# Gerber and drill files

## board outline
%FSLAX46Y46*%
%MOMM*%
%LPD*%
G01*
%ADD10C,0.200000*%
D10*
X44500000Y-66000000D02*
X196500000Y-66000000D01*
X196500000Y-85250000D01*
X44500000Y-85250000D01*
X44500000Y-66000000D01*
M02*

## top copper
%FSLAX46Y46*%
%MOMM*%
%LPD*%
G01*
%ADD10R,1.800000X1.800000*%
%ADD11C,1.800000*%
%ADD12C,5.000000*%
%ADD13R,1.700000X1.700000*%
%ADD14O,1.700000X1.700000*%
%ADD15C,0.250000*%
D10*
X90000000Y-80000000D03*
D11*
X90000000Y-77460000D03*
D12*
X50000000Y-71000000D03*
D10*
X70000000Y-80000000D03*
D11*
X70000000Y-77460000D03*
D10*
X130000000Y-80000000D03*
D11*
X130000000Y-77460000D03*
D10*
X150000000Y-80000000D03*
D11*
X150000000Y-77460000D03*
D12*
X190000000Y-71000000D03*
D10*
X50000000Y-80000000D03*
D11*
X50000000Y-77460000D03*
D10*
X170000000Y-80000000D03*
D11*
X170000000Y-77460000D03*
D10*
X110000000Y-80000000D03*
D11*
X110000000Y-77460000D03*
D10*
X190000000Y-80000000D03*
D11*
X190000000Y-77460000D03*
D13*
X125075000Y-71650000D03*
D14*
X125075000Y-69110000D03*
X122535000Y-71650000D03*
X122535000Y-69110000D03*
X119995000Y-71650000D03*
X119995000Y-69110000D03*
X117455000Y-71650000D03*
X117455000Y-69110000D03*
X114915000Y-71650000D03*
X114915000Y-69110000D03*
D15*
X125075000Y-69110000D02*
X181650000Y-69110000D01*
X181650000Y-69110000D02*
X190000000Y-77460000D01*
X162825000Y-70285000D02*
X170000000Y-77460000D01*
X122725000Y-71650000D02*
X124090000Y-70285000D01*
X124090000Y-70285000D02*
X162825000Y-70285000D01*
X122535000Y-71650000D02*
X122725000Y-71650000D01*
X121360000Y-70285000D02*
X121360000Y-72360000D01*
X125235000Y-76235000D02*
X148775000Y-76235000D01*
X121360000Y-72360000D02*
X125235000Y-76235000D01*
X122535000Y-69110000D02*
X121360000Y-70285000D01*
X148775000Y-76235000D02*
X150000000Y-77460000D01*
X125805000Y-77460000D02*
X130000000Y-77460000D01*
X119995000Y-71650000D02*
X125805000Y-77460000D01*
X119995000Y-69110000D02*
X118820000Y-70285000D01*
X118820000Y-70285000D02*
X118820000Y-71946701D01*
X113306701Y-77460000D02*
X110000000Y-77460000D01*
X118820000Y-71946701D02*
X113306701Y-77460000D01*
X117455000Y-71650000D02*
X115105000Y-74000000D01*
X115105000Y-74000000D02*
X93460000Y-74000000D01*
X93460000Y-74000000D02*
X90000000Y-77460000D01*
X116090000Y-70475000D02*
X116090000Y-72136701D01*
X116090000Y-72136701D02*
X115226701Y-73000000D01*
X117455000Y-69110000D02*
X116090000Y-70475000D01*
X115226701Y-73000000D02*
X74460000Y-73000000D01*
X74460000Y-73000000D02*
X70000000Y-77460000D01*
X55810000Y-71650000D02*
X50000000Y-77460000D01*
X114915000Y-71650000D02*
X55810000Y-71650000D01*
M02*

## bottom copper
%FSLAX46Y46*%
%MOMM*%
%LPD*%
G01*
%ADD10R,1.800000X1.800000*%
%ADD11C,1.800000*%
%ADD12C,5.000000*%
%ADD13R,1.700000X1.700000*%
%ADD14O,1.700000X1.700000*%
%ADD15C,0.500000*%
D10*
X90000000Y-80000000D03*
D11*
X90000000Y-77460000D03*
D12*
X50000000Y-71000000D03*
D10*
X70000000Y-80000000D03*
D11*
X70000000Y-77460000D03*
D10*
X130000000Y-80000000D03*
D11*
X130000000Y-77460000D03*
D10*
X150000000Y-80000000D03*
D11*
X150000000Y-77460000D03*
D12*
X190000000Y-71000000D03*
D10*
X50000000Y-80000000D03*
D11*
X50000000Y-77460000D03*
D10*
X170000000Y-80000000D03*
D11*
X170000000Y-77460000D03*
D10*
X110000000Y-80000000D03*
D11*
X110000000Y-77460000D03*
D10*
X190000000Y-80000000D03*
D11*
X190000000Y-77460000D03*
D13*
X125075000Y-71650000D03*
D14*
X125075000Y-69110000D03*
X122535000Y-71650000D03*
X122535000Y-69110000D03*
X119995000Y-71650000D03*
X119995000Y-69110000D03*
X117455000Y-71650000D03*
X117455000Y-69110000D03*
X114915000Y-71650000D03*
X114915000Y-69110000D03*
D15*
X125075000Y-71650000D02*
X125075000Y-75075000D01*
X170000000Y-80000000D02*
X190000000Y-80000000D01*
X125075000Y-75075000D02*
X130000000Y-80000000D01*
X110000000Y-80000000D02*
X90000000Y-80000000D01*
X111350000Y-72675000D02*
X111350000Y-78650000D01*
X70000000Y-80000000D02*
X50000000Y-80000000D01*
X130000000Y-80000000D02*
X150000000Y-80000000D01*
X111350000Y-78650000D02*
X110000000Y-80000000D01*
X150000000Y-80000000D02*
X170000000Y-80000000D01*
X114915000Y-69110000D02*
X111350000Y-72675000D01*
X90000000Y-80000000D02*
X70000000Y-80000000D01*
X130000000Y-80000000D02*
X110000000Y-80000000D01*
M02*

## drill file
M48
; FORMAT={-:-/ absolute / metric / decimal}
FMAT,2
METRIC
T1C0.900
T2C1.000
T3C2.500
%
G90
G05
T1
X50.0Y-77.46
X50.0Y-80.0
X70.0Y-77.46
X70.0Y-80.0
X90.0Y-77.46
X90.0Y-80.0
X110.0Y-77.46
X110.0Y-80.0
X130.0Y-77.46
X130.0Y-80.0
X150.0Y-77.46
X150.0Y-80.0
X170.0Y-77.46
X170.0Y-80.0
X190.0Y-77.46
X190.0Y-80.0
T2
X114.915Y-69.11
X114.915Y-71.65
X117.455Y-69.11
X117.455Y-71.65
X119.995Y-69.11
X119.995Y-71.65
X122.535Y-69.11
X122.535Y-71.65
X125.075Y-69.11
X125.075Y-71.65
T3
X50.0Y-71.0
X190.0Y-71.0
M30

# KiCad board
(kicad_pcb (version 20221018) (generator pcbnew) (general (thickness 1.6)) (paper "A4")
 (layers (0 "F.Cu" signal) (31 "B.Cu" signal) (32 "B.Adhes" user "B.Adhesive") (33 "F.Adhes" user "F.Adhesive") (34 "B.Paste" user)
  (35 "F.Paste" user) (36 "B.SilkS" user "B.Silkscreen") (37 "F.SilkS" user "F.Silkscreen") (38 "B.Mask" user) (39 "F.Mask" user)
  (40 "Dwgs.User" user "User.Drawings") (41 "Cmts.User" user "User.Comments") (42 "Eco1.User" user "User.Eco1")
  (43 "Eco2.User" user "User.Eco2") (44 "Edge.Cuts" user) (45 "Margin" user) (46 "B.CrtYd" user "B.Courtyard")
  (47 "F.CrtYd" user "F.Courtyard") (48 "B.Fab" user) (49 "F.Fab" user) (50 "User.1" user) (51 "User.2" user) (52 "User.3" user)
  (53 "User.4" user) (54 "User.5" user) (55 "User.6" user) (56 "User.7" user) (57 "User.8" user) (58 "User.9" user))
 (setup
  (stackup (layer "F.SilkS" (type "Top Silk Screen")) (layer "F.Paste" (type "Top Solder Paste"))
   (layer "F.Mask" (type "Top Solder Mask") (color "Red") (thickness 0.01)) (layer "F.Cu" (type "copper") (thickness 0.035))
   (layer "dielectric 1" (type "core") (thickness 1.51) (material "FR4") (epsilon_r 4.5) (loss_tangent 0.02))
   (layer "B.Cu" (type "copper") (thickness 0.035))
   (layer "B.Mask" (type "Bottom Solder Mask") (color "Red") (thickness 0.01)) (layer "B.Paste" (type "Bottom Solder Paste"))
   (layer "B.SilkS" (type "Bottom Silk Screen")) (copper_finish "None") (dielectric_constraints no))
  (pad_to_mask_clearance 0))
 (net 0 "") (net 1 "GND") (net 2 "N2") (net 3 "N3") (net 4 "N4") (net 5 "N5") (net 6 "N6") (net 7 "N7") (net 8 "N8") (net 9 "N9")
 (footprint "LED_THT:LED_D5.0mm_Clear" (layer "F.Cu") (at 90 80 90)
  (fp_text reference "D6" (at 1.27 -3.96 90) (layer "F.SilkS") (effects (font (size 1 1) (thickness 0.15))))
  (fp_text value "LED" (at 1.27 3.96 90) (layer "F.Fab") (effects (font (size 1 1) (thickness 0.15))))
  (pad "1" thru_hole rect (at 0 0 90) (size 1.8 1.8) (drill 0.9) (layers "*.Cu" "*.Mask") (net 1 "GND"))
  (pad "2" thru_hole circle (at 2.54 0 90) (size 1.8 1.8) (drill 0.9) (layers "*.Cu" "*.Mask") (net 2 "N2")))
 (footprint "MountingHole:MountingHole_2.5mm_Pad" (layer "F.Cu") (at 50 71)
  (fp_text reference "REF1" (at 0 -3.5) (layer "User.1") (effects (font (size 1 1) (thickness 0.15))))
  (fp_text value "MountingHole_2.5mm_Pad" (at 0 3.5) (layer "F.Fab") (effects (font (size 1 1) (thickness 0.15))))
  (pad "1" thru_hole circle (at 0 0) (size 5 5) (drill 2.5) (layers "*.Cu" "*.Mask")))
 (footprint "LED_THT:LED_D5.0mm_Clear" (layer "F.Cu") (at 70 80 90)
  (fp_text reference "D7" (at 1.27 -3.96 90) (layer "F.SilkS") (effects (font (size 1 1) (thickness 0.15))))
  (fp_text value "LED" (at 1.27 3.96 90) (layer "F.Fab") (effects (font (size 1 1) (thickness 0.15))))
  (pad "1" thru_hole rect (at 0 0 90) (size 1.8 1.8) (drill 0.9) (layers "*.Cu" "*.Mask") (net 1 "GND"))
  (pad "2" thru_hole circle (at 2.54 0 90) (size 1.8 1.8) (drill 0.9) (layers "*.Cu" "*.Mask") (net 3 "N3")))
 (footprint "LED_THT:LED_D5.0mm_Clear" (layer "F.Cu") (at 130 80 90)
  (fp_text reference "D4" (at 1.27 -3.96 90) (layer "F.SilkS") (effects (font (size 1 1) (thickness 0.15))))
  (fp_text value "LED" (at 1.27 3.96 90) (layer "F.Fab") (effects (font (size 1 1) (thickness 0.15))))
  (pad "1" thru_hole rect (at 0 0 90) (size 1.8 1.8) (drill 0.9) (layers "*.Cu" "*.Mask") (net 1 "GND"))
  (pad "2" thru_hole circle (at 2.54 0 90) (size 1.8 1.8) (drill 0.9) (layers "*.Cu" "*.Mask") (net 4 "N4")))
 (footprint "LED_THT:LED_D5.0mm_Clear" (layer "F.Cu") (at 150 80 90)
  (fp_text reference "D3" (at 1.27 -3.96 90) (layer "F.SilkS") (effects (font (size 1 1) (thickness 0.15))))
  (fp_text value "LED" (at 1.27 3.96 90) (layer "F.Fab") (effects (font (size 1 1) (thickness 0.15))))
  (pad "1" thru_hole rect (at 0 0 90) (size 1.8 1.8) (drill 0.9) (layers "*.Cu" "*.Mask") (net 1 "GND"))
  (pad "2" thru_hole circle (at 2.54 0 90) (size 1.8 1.8) (drill 0.9) (layers "*.Cu" "*.Mask") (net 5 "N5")))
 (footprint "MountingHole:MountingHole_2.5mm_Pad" (layer "F.Cu") (at 190 71)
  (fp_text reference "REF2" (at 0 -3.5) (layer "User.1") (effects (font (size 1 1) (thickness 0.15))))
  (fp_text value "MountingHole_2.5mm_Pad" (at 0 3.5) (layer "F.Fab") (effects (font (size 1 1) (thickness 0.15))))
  (pad "2" thru_hole circle (at 0 0) (size 5 5) (drill 2.5) (layers "*.Cu" "*.Mask")))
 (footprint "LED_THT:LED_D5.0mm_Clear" (layer "F.Cu") (at 50 80 90)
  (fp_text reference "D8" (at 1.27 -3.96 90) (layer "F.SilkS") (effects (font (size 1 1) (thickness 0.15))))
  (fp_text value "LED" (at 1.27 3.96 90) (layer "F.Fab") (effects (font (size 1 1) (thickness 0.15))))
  (pad "1" thru_hole rect (at 0 0 90) (size 1.8 1.8) (drill 0.9) (layers "*.Cu" "*.Mask") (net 1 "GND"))
  (pad "2" thru_hole circle (at 2.54 0 90) (size 1.8 1.8) (drill 0.9) (layers "*.Cu" "*.Mask") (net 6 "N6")))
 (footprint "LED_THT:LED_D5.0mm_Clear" (layer "F.Cu") (at 170 80 90)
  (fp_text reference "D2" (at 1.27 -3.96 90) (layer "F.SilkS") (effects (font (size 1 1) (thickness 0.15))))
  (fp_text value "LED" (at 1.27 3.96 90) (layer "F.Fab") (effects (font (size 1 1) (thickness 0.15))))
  (pad "1" thru_hole rect (at 0 0 90) (size 1.8 1.8) (drill 0.9) (layers "*.Cu" "*.Mask") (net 1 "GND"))
  (pad "2" thru_hole circle (at 2.54 0 90) (size 1.8 1.8) (drill 0.9) (layers "*.Cu" "*.Mask") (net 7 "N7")))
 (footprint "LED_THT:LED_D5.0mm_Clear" (layer "F.Cu") (at 110 80 90)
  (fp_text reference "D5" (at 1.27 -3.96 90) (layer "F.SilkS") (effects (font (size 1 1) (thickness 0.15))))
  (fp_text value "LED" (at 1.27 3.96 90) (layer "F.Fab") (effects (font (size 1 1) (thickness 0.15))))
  (pad "1" thru_hole rect (at 0 0 90) (size 1.8 1.8) (drill 0.9) (layers "*.Cu" "*.Mask") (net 1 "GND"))
  (pad "2" thru_hole circle (at 2.54 0 90) (size 1.8 1.8) (drill 0.9) (layers "*.Cu" "*.Mask") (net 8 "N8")))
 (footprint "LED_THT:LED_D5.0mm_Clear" (layer "F.Cu") (at 190 80 90)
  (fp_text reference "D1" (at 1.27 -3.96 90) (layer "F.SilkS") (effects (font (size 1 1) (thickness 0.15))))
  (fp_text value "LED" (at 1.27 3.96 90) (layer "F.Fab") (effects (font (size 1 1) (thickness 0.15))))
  (pad "1" thru_hole rect (at 0 0 90) (size 1.8 1.8) (drill 0.9) (layers "*.Cu" "*.Mask") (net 1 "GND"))
  (pad "2" thru_hole circle (at 2.54 0 90) (size 1.8 1.8) (drill 0.9) (layers "*.Cu" "*.Mask") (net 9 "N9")))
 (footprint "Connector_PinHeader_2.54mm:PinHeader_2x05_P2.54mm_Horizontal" (layer "B.Cu") (at 125.075 71.65 90)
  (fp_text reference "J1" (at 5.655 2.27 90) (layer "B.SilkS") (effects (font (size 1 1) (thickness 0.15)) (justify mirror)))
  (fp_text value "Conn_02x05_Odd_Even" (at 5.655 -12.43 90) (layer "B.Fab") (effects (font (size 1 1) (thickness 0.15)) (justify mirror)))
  (pad "1" thru_hole rect (at 0 0 90) (size 1.7 1.7) (drill 1) (layers "*.Cu" "*.Mask") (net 1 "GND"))
  (pad "2" thru_hole oval (at 2.54 0 90) (size 1.7 1.7) (drill 1) (layers "*.Cu" "*.Mask") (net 9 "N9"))
  (pad "3" thru_hole oval (at 0 -2.54 90) (size 1.7 1.7) (drill 1) (layers "*.Cu" "*.Mask") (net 7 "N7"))
  (pad "4" thru_hole oval (at 2.54 -2.54 90) (size 1.7 1.7) (drill 1) (layers "*.Cu" "*.Mask") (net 5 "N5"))
  (pad "5" thru_hole oval (at 0 -5.08 90) (size 1.7 1.7) (drill 1) (layers "*.Cu" "*.Mask") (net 4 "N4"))
  (pad "6" thru_hole oval (at 2.54 -5.08 90) (size 1.7 1.7) (drill 1) (layers "*.Cu" "*.Mask") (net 8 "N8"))
  (pad "7" thru_hole oval (at 0 -7.62 90) (size 1.7 1.7) (drill 1) (layers "*.Cu" "*.Mask") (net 2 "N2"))
  (pad "8" thru_hole oval (at 2.54 -7.62 90) (size 1.7 1.7) (drill 1) (layers "*.Cu" "*.Mask") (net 3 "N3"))
  (pad "9" thru_hole oval (at 0 -10.16 90) (size 1.7 1.7) (drill 1) (layers "*.Cu" "*.Mask") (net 6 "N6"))
  (pad "10" thru_hole oval (at 2.54 -10.16 90) (size 1.7 1.7) (drill 1) (layers "*.Cu" "*.Mask") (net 1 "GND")))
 (gr_rect (start 44.5 66) (end 196.5 85.25) (stroke (width 0.2) (type default)) (fill none) (layer "Edge.Cuts"))
 (segment (start 125.075 71.65) (end 125.075 75.075) (width 0.5) (layer "B.Cu") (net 1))
 (segment (start 170 80) (end 190 80) (width 0.5) (layer "B.Cu") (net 1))
 (segment (start 125.075 75.075) (end 130 80) (width 0.5) (layer "B.Cu") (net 1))
 (segment (start 110 80) (end 90 80) (width 0.5) (layer "B.Cu") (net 1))
 (segment (start 111.35 72.675) (end 111.35 78.65) (width 0.5) (layer "B.Cu") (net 1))
 (segment (start 70 80) (end 50 80) (width 0.5) (layer "B.Cu") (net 1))
 (segment (start 130 80) (end 150 80) (width 0.5) (layer "B.Cu") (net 1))
 (segment (start 111.35 78.65) (end 110 80) (width 0.5) (layer "B.Cu") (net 1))
 (segment (start 150 80) (end 170 80) (width 0.5) (layer "B.Cu") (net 1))
 (segment (start 114.915 69.11) (end 111.35 72.675) (width 0.5) (layer "B.Cu") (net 1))
 (segment (start 90 80) (end 70 80) (width 0.5) (layer "B.Cu") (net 1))
 (segment (start 130 80) (end 110 80) (width 0.5) (layer "B.Cu") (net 1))
 (segment (start 125.075 69.11) (end 181.65 69.11) (width 0.25) (layer "F.Cu") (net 9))
 (segment (start 181.65 69.11) (end 190 77.46) (width 0.25) (layer "F.Cu") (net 9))
 (segment (start 162.825 70.285) (end 170 77.46) (width 0.25) (layer "F.Cu") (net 7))
 (segment (start 122.725 71.65) (end 124.09 70.285) (width 0.25) (layer "F.Cu") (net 7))
 (segment (start 124.09 70.285) (end 162.825 70.285) (width 0.25) (layer "F.Cu") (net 7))
 (segment (start 122.535 71.65) (end 122.725 71.65) (width 0.25) (layer "F.Cu") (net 7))
 (segment (start 121.36 70.285) (end 121.36 72.36) (width 0.25) (layer "F.Cu") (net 5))
 (segment (start 125.235 76.235) (end 148.775 76.235) (width 0.25) (layer "F.Cu") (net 5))
 (segment (start 121.36 72.36) (end 125.235 76.235) (width 0.25) (layer "F.Cu") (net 5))
 (segment (start 122.535 69.11) (end 121.36 70.285) (width 0.25) (layer "F.Cu") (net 5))
 (segment (start 148.775 76.235) (end 150 77.46) (width 0.25) (layer "F.Cu") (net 5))
 (segment (start 125.805 77.46) (end 130 77.46) (width 0.25) (layer "F.Cu") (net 4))
 (segment (start 119.995 71.65) (end 125.805 77.46) (width 0.25) (layer "F.Cu") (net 4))
 (segment (start 119.995 69.11) (end 118.82 70.285) (width 0.25) (layer "F.Cu") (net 8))
 (segment (start 118.82 70.285) (end 118.82 71.946701) (width 0.25) (layer "F.Cu") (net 8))
 (segment (start 113.306701 77.46) (end 110 77.46) (width 0.25) (layer "F.Cu") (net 8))
 (segment (start 118.82 71.946701) (end 113.306701 77.46) (width 0.25) (layer "F.Cu") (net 8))
 (segment (start 117.455 71.65) (end 115.105 74) (width 0.25) (layer "F.Cu") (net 2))
 (segment (start 115.105 74) (end 93.46 74) (width 0.25) (layer "F.Cu") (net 2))
 (segment (start 93.46 74) (end 90 77.46) (width 0.25) (layer "F.Cu") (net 2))
 (segment (start 116.09 70.475) (end 116.09 72.136701) (width 0.25) (layer "F.Cu") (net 3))
 (segment (start 116.09 72.136701) (end 115.226701 73) (width 0.25) (layer "F.Cu") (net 3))
 (segment (start 117.455 69.11) (end 116.09 70.475) (width 0.25) (layer "F.Cu") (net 3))
 (segment (start 115.226701 73) (end 74.46 73) (width 0.25) (layer "F.Cu") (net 3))
 (segment (start 74.46 73) (end 70 77.46) (width 0.25) (layer "F.Cu") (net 3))
 (segment (start 55.81 71.65) (end 50 77.46) (width 0.25) (layer "F.Cu") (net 6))
 (segment (start 114.915 71.65) (end 55.81 71.65) (width 0.25) (layer "F.Cu") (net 6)))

